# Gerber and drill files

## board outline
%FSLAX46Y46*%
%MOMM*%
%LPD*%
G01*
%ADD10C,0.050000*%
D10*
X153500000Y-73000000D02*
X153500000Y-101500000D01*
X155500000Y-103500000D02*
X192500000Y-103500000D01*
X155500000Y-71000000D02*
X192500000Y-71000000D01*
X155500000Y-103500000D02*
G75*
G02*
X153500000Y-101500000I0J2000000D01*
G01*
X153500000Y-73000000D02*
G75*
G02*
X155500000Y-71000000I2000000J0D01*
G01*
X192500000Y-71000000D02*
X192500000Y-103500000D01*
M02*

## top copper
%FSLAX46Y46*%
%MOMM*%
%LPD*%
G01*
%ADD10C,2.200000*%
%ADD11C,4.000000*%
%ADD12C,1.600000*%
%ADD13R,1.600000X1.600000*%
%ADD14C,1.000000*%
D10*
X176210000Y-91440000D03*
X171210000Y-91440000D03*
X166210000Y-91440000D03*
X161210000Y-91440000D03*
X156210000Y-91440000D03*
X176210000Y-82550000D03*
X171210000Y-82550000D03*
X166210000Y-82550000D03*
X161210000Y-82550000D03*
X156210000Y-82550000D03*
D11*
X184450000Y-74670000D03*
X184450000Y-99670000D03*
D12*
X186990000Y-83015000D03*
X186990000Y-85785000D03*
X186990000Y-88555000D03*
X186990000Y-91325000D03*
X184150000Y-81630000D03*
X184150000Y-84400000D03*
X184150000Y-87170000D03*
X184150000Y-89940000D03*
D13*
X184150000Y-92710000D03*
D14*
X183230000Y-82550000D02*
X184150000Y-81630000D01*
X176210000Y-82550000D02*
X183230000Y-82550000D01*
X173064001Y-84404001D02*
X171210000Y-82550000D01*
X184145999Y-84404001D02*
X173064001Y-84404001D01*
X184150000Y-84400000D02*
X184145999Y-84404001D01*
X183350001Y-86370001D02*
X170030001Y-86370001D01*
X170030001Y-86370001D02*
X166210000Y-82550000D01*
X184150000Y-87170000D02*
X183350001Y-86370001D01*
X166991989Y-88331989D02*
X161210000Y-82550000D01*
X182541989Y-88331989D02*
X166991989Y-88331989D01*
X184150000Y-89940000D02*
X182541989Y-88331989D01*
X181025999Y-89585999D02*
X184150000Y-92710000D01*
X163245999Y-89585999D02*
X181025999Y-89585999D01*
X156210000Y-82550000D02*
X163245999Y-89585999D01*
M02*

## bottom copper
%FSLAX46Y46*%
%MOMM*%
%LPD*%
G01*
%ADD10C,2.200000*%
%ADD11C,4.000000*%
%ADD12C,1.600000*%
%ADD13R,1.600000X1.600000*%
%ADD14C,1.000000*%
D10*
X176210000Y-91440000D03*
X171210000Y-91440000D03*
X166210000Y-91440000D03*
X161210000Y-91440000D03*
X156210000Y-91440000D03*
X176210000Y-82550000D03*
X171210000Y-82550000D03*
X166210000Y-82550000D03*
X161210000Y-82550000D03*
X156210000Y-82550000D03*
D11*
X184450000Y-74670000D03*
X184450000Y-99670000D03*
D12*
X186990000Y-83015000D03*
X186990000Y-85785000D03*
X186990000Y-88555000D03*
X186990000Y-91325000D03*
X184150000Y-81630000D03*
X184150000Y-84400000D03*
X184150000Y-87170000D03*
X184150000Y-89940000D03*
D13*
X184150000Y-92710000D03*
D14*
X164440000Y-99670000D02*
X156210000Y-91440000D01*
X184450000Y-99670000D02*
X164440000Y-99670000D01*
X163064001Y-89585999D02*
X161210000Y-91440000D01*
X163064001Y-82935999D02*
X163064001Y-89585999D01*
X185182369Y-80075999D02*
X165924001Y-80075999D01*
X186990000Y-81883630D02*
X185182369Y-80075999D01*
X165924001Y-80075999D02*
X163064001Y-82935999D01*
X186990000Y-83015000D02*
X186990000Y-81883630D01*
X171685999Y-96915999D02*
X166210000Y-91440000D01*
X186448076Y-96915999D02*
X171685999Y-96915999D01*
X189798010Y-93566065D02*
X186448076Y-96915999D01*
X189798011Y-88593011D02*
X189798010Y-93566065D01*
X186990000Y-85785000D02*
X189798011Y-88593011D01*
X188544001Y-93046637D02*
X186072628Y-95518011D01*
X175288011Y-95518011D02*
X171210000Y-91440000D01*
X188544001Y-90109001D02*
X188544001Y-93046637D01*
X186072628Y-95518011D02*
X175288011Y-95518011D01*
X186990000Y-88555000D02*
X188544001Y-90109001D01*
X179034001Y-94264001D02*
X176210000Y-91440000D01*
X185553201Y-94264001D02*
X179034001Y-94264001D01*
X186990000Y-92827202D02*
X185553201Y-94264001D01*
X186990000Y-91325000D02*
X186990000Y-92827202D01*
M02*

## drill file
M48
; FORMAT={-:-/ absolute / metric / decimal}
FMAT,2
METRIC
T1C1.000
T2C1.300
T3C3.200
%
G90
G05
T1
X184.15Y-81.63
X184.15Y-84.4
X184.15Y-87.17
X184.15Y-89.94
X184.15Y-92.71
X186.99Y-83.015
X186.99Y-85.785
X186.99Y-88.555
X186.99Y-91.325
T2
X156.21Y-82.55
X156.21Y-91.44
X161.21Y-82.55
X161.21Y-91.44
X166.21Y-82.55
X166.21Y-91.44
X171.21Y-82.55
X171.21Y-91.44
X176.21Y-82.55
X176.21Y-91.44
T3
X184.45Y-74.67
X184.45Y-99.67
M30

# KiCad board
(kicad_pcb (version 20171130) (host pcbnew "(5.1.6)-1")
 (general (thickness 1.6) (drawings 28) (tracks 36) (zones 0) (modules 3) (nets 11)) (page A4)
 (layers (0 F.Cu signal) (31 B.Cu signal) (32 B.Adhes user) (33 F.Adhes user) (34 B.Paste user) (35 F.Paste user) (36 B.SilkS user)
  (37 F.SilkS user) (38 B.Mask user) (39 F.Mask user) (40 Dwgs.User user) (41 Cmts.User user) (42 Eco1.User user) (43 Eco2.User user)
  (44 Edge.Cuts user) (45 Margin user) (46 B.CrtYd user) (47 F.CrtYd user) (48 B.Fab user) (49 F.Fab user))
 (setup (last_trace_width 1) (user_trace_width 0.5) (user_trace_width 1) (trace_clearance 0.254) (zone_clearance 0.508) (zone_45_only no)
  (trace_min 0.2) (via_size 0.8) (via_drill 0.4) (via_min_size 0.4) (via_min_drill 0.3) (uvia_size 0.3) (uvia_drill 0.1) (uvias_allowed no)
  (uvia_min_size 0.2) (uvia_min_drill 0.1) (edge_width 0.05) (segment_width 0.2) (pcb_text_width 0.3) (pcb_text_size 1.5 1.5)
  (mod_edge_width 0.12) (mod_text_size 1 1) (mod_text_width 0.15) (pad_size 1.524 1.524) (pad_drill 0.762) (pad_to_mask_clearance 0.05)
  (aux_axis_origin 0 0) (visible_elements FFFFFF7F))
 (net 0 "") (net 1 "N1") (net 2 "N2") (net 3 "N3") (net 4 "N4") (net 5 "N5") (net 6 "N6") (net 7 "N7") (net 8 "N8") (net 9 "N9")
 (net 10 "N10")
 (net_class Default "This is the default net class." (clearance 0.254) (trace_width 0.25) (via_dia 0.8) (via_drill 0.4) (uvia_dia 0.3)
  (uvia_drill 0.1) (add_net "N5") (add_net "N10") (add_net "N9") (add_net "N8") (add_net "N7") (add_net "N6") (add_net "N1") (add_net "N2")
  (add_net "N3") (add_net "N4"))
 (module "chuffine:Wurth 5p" (layer F.Cu) (at 156.21 91.44)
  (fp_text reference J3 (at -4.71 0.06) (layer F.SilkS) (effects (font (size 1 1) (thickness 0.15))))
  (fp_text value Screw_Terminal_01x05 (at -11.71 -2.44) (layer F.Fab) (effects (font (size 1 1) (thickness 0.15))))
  (pad 5 thru_hole circle (at 20 0) (size 2.2 2.2) (drill 1.3) (layers *.Cu *.Mask) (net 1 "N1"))
  (pad 4 thru_hole circle (at 15 0) (size 2.2 2.2) (drill 1.3) (layers *.Cu *.Mask) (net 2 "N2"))
  (pad 3 thru_hole circle (at 10 0) (size 2.2 2.2) (drill 1.3) (layers *.Cu *.Mask) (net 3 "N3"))
  (pad 2 thru_hole circle (at 5 0) (size 2.2 2.2) (drill 1.3) (layers *.Cu *.Mask) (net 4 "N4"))
  (pad 1 thru_hole circle (at 0 0) (size 2.2 2.2) (drill 1.3) (layers *.Cu *.Mask) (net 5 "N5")))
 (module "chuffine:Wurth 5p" (layer F.Cu) (at 156.21 82.55)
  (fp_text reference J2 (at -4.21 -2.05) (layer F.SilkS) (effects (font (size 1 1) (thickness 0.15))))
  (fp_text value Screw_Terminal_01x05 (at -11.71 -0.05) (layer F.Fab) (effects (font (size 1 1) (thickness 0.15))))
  (pad 5 thru_hole circle (at 20 0) (size 2.2 2.2) (drill 1.3) (layers *.Cu *.Mask) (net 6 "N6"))
  (pad 4 thru_hole circle (at 15 0) (size 2.2 2.2) (drill 1.3) (layers *.Cu *.Mask) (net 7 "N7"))
  (pad 3 thru_hole circle (at 10 0) (size 2.2 2.2) (drill 1.3) (layers *.Cu *.Mask) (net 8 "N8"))
  (pad 2 thru_hole circle (at 5 0) (size 2.2 2.2) (drill 1.3) (layers *.Cu *.Mask) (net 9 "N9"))
  (pad 1 thru_hole circle (at 0 0) (size 2.2 2.2) (drill 1.3) (layers *.Cu *.Mask) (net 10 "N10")))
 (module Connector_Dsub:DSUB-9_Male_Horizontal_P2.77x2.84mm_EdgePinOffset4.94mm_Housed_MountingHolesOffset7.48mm (layer F.Cu)
  (at 184.15 92.71 90)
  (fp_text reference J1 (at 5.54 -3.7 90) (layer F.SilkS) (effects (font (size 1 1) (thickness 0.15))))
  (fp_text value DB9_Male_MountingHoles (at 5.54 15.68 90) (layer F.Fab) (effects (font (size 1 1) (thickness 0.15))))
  (pad 0 thru_hole circle (at 18.04 0.3 90) (size 4 4) (drill 3.2) (layers *.Cu *.Mask) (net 5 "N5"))
  (pad 0 thru_hole circle (at -6.96 0.3 90) (size 4 4) (drill 3.2) (layers *.Cu *.Mask) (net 5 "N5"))
  (pad 9 thru_hole circle (at 9.695 2.84 90) (size 1.6 1.6) (drill 1) (layers *.Cu *.Mask) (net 4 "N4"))
  (pad 8 thru_hole circle (at 6.925 2.84 90) (size 1.6 1.6) (drill 1) (layers *.Cu *.Mask) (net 3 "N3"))
  (pad 7 thru_hole circle (at 4.155 2.84 90) (size 1.6 1.6) (drill 1) (layers *.Cu *.Mask) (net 2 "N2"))
  (pad 6 thru_hole circle (at 1.385 2.84 90) (size 1.6 1.6) (drill 1) (layers *.Cu *.Mask) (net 1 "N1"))
  (pad 5 thru_hole circle (at 11.08 0 90) (size 1.6 1.6) (drill 1) (layers *.Cu *.Mask) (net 6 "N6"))
  (pad 4 thru_hole circle (at 8.31 0 90) (size 1.6 1.6) (drill 1) (layers *.Cu *.Mask) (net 7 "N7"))
  (pad 3 thru_hole circle (at 5.54 0 90) (size 1.6 1.6) (drill 1) (layers *.Cu *.Mask) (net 8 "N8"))
  (pad 2 thru_hole circle (at 2.77 0 90) (size 1.6 1.6) (drill 1) (layers *.Cu *.Mask) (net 9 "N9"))
  (pad 1 thru_hole rect (at 0 0 90) (size 1.6 1.6) (drill 1) (layers *.Cu *.Mask) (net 10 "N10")))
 (gr_line (start 153.5 73) (end 153.5 101.5) (layer Edge.Cuts) (width 0.05))
 (gr_line (start 155.5 103.5) (end 192.5 103.5) (layer Edge.Cuts) (width 0.05))
 (gr_line (start 155.5 71) (end 192.5 71) (layer Edge.Cuts) (width 0.05))
 (gr_arc (start 155.5 101.5) (end 153.5 101.5) (angle -90) (layer Edge.Cuts) (width 0.05))
 (gr_arc (start 155.5 73) (end 155.5 71) (angle -90) (layer Edge.Cuts) (width 0.05))
 (gr_line (start 192.5 71) (end 192.5 103.5) (layer Edge.Cuts) (width 0.05))
 (segment (start 164.44 99.67) (end 156.21 91.44) (width 1) (layer B.Cu) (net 5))
 (segment (start 184.45 99.67) (end 164.44 99.67) (width 1) (layer B.Cu) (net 5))
 (segment (start 163.064001 89.585999) (end 161.21 91.44) (width 1) (layer B.Cu) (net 4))
 (segment (start 163.064001 82.935999) (end 163.064001 89.585999) (width 1) (layer B.Cu) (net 4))
 (segment (start 185.182369 80.075999) (end 165.924001 80.075999) (width 1) (layer B.Cu) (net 4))
 (segment (start 186.99 81.88363) (end 185.182369 80.075999) (width 1) (layer B.Cu) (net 4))
 (segment (start 165.924001 80.075999) (end 163.064001 82.935999) (width 1) (layer B.Cu) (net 4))
 (segment (start 186.99 83.015) (end 186.99 81.88363) (width 1) (layer B.Cu) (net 4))
 (segment (start 171.685999 96.915999) (end 166.21 91.44) (width 1) (layer B.Cu) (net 3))
 (segment (start 186.448076 96.915999) (end 171.685999 96.915999) (width 1) (layer B.Cu) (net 3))
 (segment (start 189.79801 93.566065) (end 186.448076 96.915999) (width 1) (layer B.Cu) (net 3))
 (segment (start 189.798011 88.593011) (end 189.79801 93.566065) (width 1) (layer B.Cu) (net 3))
 (segment (start 186.99 85.785) (end 189.798011 88.593011) (width 1) (layer B.Cu) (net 3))
 (segment (start 188.544001 93.046637) (end 186.072628 95.518011) (width 1) (layer B.Cu) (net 2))
 (segment (start 175.288011 95.518011) (end 171.21 91.44) (width 1) (layer B.Cu) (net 2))
 (segment (start 188.544001 90.109001) (end 188.544001 93.046637) (width 1) (layer B.Cu) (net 2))
 (segment (start 186.072628 95.518011) (end 175.288011 95.518011) (width 1) (layer B.Cu) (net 2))
 (segment (start 186.99 88.555) (end 188.544001 90.109001) (width 1) (layer B.Cu) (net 2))
 (segment (start 179.034001 94.264001) (end 176.21 91.44) (width 1) (layer B.Cu) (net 1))
 (segment (start 185.553201 94.264001) (end 179.034001 94.264001) (width 1) (layer B.Cu) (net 1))
 (segment (start 186.99 92.827202) (end 185.553201 94.264001) (width 1) (layer B.Cu) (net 1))
 (segment (start 186.99 91.325) (end 186.99 92.827202) (width 1) (layer B.Cu) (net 1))
 (segment (start 183.23 82.55) (end 184.15 81.63) (width 1) (layer F.Cu) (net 6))
 (segment (start 176.21 82.55) (end 183.23 82.55) (width 1) (layer F.Cu) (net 6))
 (segment (start 173.064001 84.404001) (end 171.21 82.55) (width 1) (layer F.Cu) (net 7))
 (segment (start 184.145999 84.404001) (end 173.064001 84.404001) (width 1) (layer F.Cu) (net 7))
 (segment (start 184.15 84.4) (end 184.145999 84.404001) (width 1) (layer F.Cu) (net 7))
 (segment (start 183.350001 86.370001) (end 170.030001 86.370001) (width 1) (layer F.Cu) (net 8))
 (segment (start 170.030001 86.370001) (end 166.21 82.55) (width 1) (layer F.Cu) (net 8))
 (segment (start 184.15 87.17) (end 183.350001 86.370001) (width 1) (layer F.Cu) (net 8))
 (segment (start 166.991989 88.331989) (end 161.21 82.55) (width 1) (layer F.Cu) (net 9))
 (segment (start 182.541989 88.331989) (end 166.991989 88.331989) (width 1) (layer F.Cu) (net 9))
 (segment (start 184.15 89.94) (end 182.541989 88.331989) (width 1) (layer F.Cu) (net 9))
 (segment (start 181.025999 89.585999) (end 184.15 92.71) (width 1) (layer F.Cu) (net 10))
 (segment (start 163.245999 89.585999) (end 181.025999 89.585999) (width 1) (layer F.Cu) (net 10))
 (segment (start 156.21 82.55) (end 163.245999 89.585999) (width 1) (layer F.Cu) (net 10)))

